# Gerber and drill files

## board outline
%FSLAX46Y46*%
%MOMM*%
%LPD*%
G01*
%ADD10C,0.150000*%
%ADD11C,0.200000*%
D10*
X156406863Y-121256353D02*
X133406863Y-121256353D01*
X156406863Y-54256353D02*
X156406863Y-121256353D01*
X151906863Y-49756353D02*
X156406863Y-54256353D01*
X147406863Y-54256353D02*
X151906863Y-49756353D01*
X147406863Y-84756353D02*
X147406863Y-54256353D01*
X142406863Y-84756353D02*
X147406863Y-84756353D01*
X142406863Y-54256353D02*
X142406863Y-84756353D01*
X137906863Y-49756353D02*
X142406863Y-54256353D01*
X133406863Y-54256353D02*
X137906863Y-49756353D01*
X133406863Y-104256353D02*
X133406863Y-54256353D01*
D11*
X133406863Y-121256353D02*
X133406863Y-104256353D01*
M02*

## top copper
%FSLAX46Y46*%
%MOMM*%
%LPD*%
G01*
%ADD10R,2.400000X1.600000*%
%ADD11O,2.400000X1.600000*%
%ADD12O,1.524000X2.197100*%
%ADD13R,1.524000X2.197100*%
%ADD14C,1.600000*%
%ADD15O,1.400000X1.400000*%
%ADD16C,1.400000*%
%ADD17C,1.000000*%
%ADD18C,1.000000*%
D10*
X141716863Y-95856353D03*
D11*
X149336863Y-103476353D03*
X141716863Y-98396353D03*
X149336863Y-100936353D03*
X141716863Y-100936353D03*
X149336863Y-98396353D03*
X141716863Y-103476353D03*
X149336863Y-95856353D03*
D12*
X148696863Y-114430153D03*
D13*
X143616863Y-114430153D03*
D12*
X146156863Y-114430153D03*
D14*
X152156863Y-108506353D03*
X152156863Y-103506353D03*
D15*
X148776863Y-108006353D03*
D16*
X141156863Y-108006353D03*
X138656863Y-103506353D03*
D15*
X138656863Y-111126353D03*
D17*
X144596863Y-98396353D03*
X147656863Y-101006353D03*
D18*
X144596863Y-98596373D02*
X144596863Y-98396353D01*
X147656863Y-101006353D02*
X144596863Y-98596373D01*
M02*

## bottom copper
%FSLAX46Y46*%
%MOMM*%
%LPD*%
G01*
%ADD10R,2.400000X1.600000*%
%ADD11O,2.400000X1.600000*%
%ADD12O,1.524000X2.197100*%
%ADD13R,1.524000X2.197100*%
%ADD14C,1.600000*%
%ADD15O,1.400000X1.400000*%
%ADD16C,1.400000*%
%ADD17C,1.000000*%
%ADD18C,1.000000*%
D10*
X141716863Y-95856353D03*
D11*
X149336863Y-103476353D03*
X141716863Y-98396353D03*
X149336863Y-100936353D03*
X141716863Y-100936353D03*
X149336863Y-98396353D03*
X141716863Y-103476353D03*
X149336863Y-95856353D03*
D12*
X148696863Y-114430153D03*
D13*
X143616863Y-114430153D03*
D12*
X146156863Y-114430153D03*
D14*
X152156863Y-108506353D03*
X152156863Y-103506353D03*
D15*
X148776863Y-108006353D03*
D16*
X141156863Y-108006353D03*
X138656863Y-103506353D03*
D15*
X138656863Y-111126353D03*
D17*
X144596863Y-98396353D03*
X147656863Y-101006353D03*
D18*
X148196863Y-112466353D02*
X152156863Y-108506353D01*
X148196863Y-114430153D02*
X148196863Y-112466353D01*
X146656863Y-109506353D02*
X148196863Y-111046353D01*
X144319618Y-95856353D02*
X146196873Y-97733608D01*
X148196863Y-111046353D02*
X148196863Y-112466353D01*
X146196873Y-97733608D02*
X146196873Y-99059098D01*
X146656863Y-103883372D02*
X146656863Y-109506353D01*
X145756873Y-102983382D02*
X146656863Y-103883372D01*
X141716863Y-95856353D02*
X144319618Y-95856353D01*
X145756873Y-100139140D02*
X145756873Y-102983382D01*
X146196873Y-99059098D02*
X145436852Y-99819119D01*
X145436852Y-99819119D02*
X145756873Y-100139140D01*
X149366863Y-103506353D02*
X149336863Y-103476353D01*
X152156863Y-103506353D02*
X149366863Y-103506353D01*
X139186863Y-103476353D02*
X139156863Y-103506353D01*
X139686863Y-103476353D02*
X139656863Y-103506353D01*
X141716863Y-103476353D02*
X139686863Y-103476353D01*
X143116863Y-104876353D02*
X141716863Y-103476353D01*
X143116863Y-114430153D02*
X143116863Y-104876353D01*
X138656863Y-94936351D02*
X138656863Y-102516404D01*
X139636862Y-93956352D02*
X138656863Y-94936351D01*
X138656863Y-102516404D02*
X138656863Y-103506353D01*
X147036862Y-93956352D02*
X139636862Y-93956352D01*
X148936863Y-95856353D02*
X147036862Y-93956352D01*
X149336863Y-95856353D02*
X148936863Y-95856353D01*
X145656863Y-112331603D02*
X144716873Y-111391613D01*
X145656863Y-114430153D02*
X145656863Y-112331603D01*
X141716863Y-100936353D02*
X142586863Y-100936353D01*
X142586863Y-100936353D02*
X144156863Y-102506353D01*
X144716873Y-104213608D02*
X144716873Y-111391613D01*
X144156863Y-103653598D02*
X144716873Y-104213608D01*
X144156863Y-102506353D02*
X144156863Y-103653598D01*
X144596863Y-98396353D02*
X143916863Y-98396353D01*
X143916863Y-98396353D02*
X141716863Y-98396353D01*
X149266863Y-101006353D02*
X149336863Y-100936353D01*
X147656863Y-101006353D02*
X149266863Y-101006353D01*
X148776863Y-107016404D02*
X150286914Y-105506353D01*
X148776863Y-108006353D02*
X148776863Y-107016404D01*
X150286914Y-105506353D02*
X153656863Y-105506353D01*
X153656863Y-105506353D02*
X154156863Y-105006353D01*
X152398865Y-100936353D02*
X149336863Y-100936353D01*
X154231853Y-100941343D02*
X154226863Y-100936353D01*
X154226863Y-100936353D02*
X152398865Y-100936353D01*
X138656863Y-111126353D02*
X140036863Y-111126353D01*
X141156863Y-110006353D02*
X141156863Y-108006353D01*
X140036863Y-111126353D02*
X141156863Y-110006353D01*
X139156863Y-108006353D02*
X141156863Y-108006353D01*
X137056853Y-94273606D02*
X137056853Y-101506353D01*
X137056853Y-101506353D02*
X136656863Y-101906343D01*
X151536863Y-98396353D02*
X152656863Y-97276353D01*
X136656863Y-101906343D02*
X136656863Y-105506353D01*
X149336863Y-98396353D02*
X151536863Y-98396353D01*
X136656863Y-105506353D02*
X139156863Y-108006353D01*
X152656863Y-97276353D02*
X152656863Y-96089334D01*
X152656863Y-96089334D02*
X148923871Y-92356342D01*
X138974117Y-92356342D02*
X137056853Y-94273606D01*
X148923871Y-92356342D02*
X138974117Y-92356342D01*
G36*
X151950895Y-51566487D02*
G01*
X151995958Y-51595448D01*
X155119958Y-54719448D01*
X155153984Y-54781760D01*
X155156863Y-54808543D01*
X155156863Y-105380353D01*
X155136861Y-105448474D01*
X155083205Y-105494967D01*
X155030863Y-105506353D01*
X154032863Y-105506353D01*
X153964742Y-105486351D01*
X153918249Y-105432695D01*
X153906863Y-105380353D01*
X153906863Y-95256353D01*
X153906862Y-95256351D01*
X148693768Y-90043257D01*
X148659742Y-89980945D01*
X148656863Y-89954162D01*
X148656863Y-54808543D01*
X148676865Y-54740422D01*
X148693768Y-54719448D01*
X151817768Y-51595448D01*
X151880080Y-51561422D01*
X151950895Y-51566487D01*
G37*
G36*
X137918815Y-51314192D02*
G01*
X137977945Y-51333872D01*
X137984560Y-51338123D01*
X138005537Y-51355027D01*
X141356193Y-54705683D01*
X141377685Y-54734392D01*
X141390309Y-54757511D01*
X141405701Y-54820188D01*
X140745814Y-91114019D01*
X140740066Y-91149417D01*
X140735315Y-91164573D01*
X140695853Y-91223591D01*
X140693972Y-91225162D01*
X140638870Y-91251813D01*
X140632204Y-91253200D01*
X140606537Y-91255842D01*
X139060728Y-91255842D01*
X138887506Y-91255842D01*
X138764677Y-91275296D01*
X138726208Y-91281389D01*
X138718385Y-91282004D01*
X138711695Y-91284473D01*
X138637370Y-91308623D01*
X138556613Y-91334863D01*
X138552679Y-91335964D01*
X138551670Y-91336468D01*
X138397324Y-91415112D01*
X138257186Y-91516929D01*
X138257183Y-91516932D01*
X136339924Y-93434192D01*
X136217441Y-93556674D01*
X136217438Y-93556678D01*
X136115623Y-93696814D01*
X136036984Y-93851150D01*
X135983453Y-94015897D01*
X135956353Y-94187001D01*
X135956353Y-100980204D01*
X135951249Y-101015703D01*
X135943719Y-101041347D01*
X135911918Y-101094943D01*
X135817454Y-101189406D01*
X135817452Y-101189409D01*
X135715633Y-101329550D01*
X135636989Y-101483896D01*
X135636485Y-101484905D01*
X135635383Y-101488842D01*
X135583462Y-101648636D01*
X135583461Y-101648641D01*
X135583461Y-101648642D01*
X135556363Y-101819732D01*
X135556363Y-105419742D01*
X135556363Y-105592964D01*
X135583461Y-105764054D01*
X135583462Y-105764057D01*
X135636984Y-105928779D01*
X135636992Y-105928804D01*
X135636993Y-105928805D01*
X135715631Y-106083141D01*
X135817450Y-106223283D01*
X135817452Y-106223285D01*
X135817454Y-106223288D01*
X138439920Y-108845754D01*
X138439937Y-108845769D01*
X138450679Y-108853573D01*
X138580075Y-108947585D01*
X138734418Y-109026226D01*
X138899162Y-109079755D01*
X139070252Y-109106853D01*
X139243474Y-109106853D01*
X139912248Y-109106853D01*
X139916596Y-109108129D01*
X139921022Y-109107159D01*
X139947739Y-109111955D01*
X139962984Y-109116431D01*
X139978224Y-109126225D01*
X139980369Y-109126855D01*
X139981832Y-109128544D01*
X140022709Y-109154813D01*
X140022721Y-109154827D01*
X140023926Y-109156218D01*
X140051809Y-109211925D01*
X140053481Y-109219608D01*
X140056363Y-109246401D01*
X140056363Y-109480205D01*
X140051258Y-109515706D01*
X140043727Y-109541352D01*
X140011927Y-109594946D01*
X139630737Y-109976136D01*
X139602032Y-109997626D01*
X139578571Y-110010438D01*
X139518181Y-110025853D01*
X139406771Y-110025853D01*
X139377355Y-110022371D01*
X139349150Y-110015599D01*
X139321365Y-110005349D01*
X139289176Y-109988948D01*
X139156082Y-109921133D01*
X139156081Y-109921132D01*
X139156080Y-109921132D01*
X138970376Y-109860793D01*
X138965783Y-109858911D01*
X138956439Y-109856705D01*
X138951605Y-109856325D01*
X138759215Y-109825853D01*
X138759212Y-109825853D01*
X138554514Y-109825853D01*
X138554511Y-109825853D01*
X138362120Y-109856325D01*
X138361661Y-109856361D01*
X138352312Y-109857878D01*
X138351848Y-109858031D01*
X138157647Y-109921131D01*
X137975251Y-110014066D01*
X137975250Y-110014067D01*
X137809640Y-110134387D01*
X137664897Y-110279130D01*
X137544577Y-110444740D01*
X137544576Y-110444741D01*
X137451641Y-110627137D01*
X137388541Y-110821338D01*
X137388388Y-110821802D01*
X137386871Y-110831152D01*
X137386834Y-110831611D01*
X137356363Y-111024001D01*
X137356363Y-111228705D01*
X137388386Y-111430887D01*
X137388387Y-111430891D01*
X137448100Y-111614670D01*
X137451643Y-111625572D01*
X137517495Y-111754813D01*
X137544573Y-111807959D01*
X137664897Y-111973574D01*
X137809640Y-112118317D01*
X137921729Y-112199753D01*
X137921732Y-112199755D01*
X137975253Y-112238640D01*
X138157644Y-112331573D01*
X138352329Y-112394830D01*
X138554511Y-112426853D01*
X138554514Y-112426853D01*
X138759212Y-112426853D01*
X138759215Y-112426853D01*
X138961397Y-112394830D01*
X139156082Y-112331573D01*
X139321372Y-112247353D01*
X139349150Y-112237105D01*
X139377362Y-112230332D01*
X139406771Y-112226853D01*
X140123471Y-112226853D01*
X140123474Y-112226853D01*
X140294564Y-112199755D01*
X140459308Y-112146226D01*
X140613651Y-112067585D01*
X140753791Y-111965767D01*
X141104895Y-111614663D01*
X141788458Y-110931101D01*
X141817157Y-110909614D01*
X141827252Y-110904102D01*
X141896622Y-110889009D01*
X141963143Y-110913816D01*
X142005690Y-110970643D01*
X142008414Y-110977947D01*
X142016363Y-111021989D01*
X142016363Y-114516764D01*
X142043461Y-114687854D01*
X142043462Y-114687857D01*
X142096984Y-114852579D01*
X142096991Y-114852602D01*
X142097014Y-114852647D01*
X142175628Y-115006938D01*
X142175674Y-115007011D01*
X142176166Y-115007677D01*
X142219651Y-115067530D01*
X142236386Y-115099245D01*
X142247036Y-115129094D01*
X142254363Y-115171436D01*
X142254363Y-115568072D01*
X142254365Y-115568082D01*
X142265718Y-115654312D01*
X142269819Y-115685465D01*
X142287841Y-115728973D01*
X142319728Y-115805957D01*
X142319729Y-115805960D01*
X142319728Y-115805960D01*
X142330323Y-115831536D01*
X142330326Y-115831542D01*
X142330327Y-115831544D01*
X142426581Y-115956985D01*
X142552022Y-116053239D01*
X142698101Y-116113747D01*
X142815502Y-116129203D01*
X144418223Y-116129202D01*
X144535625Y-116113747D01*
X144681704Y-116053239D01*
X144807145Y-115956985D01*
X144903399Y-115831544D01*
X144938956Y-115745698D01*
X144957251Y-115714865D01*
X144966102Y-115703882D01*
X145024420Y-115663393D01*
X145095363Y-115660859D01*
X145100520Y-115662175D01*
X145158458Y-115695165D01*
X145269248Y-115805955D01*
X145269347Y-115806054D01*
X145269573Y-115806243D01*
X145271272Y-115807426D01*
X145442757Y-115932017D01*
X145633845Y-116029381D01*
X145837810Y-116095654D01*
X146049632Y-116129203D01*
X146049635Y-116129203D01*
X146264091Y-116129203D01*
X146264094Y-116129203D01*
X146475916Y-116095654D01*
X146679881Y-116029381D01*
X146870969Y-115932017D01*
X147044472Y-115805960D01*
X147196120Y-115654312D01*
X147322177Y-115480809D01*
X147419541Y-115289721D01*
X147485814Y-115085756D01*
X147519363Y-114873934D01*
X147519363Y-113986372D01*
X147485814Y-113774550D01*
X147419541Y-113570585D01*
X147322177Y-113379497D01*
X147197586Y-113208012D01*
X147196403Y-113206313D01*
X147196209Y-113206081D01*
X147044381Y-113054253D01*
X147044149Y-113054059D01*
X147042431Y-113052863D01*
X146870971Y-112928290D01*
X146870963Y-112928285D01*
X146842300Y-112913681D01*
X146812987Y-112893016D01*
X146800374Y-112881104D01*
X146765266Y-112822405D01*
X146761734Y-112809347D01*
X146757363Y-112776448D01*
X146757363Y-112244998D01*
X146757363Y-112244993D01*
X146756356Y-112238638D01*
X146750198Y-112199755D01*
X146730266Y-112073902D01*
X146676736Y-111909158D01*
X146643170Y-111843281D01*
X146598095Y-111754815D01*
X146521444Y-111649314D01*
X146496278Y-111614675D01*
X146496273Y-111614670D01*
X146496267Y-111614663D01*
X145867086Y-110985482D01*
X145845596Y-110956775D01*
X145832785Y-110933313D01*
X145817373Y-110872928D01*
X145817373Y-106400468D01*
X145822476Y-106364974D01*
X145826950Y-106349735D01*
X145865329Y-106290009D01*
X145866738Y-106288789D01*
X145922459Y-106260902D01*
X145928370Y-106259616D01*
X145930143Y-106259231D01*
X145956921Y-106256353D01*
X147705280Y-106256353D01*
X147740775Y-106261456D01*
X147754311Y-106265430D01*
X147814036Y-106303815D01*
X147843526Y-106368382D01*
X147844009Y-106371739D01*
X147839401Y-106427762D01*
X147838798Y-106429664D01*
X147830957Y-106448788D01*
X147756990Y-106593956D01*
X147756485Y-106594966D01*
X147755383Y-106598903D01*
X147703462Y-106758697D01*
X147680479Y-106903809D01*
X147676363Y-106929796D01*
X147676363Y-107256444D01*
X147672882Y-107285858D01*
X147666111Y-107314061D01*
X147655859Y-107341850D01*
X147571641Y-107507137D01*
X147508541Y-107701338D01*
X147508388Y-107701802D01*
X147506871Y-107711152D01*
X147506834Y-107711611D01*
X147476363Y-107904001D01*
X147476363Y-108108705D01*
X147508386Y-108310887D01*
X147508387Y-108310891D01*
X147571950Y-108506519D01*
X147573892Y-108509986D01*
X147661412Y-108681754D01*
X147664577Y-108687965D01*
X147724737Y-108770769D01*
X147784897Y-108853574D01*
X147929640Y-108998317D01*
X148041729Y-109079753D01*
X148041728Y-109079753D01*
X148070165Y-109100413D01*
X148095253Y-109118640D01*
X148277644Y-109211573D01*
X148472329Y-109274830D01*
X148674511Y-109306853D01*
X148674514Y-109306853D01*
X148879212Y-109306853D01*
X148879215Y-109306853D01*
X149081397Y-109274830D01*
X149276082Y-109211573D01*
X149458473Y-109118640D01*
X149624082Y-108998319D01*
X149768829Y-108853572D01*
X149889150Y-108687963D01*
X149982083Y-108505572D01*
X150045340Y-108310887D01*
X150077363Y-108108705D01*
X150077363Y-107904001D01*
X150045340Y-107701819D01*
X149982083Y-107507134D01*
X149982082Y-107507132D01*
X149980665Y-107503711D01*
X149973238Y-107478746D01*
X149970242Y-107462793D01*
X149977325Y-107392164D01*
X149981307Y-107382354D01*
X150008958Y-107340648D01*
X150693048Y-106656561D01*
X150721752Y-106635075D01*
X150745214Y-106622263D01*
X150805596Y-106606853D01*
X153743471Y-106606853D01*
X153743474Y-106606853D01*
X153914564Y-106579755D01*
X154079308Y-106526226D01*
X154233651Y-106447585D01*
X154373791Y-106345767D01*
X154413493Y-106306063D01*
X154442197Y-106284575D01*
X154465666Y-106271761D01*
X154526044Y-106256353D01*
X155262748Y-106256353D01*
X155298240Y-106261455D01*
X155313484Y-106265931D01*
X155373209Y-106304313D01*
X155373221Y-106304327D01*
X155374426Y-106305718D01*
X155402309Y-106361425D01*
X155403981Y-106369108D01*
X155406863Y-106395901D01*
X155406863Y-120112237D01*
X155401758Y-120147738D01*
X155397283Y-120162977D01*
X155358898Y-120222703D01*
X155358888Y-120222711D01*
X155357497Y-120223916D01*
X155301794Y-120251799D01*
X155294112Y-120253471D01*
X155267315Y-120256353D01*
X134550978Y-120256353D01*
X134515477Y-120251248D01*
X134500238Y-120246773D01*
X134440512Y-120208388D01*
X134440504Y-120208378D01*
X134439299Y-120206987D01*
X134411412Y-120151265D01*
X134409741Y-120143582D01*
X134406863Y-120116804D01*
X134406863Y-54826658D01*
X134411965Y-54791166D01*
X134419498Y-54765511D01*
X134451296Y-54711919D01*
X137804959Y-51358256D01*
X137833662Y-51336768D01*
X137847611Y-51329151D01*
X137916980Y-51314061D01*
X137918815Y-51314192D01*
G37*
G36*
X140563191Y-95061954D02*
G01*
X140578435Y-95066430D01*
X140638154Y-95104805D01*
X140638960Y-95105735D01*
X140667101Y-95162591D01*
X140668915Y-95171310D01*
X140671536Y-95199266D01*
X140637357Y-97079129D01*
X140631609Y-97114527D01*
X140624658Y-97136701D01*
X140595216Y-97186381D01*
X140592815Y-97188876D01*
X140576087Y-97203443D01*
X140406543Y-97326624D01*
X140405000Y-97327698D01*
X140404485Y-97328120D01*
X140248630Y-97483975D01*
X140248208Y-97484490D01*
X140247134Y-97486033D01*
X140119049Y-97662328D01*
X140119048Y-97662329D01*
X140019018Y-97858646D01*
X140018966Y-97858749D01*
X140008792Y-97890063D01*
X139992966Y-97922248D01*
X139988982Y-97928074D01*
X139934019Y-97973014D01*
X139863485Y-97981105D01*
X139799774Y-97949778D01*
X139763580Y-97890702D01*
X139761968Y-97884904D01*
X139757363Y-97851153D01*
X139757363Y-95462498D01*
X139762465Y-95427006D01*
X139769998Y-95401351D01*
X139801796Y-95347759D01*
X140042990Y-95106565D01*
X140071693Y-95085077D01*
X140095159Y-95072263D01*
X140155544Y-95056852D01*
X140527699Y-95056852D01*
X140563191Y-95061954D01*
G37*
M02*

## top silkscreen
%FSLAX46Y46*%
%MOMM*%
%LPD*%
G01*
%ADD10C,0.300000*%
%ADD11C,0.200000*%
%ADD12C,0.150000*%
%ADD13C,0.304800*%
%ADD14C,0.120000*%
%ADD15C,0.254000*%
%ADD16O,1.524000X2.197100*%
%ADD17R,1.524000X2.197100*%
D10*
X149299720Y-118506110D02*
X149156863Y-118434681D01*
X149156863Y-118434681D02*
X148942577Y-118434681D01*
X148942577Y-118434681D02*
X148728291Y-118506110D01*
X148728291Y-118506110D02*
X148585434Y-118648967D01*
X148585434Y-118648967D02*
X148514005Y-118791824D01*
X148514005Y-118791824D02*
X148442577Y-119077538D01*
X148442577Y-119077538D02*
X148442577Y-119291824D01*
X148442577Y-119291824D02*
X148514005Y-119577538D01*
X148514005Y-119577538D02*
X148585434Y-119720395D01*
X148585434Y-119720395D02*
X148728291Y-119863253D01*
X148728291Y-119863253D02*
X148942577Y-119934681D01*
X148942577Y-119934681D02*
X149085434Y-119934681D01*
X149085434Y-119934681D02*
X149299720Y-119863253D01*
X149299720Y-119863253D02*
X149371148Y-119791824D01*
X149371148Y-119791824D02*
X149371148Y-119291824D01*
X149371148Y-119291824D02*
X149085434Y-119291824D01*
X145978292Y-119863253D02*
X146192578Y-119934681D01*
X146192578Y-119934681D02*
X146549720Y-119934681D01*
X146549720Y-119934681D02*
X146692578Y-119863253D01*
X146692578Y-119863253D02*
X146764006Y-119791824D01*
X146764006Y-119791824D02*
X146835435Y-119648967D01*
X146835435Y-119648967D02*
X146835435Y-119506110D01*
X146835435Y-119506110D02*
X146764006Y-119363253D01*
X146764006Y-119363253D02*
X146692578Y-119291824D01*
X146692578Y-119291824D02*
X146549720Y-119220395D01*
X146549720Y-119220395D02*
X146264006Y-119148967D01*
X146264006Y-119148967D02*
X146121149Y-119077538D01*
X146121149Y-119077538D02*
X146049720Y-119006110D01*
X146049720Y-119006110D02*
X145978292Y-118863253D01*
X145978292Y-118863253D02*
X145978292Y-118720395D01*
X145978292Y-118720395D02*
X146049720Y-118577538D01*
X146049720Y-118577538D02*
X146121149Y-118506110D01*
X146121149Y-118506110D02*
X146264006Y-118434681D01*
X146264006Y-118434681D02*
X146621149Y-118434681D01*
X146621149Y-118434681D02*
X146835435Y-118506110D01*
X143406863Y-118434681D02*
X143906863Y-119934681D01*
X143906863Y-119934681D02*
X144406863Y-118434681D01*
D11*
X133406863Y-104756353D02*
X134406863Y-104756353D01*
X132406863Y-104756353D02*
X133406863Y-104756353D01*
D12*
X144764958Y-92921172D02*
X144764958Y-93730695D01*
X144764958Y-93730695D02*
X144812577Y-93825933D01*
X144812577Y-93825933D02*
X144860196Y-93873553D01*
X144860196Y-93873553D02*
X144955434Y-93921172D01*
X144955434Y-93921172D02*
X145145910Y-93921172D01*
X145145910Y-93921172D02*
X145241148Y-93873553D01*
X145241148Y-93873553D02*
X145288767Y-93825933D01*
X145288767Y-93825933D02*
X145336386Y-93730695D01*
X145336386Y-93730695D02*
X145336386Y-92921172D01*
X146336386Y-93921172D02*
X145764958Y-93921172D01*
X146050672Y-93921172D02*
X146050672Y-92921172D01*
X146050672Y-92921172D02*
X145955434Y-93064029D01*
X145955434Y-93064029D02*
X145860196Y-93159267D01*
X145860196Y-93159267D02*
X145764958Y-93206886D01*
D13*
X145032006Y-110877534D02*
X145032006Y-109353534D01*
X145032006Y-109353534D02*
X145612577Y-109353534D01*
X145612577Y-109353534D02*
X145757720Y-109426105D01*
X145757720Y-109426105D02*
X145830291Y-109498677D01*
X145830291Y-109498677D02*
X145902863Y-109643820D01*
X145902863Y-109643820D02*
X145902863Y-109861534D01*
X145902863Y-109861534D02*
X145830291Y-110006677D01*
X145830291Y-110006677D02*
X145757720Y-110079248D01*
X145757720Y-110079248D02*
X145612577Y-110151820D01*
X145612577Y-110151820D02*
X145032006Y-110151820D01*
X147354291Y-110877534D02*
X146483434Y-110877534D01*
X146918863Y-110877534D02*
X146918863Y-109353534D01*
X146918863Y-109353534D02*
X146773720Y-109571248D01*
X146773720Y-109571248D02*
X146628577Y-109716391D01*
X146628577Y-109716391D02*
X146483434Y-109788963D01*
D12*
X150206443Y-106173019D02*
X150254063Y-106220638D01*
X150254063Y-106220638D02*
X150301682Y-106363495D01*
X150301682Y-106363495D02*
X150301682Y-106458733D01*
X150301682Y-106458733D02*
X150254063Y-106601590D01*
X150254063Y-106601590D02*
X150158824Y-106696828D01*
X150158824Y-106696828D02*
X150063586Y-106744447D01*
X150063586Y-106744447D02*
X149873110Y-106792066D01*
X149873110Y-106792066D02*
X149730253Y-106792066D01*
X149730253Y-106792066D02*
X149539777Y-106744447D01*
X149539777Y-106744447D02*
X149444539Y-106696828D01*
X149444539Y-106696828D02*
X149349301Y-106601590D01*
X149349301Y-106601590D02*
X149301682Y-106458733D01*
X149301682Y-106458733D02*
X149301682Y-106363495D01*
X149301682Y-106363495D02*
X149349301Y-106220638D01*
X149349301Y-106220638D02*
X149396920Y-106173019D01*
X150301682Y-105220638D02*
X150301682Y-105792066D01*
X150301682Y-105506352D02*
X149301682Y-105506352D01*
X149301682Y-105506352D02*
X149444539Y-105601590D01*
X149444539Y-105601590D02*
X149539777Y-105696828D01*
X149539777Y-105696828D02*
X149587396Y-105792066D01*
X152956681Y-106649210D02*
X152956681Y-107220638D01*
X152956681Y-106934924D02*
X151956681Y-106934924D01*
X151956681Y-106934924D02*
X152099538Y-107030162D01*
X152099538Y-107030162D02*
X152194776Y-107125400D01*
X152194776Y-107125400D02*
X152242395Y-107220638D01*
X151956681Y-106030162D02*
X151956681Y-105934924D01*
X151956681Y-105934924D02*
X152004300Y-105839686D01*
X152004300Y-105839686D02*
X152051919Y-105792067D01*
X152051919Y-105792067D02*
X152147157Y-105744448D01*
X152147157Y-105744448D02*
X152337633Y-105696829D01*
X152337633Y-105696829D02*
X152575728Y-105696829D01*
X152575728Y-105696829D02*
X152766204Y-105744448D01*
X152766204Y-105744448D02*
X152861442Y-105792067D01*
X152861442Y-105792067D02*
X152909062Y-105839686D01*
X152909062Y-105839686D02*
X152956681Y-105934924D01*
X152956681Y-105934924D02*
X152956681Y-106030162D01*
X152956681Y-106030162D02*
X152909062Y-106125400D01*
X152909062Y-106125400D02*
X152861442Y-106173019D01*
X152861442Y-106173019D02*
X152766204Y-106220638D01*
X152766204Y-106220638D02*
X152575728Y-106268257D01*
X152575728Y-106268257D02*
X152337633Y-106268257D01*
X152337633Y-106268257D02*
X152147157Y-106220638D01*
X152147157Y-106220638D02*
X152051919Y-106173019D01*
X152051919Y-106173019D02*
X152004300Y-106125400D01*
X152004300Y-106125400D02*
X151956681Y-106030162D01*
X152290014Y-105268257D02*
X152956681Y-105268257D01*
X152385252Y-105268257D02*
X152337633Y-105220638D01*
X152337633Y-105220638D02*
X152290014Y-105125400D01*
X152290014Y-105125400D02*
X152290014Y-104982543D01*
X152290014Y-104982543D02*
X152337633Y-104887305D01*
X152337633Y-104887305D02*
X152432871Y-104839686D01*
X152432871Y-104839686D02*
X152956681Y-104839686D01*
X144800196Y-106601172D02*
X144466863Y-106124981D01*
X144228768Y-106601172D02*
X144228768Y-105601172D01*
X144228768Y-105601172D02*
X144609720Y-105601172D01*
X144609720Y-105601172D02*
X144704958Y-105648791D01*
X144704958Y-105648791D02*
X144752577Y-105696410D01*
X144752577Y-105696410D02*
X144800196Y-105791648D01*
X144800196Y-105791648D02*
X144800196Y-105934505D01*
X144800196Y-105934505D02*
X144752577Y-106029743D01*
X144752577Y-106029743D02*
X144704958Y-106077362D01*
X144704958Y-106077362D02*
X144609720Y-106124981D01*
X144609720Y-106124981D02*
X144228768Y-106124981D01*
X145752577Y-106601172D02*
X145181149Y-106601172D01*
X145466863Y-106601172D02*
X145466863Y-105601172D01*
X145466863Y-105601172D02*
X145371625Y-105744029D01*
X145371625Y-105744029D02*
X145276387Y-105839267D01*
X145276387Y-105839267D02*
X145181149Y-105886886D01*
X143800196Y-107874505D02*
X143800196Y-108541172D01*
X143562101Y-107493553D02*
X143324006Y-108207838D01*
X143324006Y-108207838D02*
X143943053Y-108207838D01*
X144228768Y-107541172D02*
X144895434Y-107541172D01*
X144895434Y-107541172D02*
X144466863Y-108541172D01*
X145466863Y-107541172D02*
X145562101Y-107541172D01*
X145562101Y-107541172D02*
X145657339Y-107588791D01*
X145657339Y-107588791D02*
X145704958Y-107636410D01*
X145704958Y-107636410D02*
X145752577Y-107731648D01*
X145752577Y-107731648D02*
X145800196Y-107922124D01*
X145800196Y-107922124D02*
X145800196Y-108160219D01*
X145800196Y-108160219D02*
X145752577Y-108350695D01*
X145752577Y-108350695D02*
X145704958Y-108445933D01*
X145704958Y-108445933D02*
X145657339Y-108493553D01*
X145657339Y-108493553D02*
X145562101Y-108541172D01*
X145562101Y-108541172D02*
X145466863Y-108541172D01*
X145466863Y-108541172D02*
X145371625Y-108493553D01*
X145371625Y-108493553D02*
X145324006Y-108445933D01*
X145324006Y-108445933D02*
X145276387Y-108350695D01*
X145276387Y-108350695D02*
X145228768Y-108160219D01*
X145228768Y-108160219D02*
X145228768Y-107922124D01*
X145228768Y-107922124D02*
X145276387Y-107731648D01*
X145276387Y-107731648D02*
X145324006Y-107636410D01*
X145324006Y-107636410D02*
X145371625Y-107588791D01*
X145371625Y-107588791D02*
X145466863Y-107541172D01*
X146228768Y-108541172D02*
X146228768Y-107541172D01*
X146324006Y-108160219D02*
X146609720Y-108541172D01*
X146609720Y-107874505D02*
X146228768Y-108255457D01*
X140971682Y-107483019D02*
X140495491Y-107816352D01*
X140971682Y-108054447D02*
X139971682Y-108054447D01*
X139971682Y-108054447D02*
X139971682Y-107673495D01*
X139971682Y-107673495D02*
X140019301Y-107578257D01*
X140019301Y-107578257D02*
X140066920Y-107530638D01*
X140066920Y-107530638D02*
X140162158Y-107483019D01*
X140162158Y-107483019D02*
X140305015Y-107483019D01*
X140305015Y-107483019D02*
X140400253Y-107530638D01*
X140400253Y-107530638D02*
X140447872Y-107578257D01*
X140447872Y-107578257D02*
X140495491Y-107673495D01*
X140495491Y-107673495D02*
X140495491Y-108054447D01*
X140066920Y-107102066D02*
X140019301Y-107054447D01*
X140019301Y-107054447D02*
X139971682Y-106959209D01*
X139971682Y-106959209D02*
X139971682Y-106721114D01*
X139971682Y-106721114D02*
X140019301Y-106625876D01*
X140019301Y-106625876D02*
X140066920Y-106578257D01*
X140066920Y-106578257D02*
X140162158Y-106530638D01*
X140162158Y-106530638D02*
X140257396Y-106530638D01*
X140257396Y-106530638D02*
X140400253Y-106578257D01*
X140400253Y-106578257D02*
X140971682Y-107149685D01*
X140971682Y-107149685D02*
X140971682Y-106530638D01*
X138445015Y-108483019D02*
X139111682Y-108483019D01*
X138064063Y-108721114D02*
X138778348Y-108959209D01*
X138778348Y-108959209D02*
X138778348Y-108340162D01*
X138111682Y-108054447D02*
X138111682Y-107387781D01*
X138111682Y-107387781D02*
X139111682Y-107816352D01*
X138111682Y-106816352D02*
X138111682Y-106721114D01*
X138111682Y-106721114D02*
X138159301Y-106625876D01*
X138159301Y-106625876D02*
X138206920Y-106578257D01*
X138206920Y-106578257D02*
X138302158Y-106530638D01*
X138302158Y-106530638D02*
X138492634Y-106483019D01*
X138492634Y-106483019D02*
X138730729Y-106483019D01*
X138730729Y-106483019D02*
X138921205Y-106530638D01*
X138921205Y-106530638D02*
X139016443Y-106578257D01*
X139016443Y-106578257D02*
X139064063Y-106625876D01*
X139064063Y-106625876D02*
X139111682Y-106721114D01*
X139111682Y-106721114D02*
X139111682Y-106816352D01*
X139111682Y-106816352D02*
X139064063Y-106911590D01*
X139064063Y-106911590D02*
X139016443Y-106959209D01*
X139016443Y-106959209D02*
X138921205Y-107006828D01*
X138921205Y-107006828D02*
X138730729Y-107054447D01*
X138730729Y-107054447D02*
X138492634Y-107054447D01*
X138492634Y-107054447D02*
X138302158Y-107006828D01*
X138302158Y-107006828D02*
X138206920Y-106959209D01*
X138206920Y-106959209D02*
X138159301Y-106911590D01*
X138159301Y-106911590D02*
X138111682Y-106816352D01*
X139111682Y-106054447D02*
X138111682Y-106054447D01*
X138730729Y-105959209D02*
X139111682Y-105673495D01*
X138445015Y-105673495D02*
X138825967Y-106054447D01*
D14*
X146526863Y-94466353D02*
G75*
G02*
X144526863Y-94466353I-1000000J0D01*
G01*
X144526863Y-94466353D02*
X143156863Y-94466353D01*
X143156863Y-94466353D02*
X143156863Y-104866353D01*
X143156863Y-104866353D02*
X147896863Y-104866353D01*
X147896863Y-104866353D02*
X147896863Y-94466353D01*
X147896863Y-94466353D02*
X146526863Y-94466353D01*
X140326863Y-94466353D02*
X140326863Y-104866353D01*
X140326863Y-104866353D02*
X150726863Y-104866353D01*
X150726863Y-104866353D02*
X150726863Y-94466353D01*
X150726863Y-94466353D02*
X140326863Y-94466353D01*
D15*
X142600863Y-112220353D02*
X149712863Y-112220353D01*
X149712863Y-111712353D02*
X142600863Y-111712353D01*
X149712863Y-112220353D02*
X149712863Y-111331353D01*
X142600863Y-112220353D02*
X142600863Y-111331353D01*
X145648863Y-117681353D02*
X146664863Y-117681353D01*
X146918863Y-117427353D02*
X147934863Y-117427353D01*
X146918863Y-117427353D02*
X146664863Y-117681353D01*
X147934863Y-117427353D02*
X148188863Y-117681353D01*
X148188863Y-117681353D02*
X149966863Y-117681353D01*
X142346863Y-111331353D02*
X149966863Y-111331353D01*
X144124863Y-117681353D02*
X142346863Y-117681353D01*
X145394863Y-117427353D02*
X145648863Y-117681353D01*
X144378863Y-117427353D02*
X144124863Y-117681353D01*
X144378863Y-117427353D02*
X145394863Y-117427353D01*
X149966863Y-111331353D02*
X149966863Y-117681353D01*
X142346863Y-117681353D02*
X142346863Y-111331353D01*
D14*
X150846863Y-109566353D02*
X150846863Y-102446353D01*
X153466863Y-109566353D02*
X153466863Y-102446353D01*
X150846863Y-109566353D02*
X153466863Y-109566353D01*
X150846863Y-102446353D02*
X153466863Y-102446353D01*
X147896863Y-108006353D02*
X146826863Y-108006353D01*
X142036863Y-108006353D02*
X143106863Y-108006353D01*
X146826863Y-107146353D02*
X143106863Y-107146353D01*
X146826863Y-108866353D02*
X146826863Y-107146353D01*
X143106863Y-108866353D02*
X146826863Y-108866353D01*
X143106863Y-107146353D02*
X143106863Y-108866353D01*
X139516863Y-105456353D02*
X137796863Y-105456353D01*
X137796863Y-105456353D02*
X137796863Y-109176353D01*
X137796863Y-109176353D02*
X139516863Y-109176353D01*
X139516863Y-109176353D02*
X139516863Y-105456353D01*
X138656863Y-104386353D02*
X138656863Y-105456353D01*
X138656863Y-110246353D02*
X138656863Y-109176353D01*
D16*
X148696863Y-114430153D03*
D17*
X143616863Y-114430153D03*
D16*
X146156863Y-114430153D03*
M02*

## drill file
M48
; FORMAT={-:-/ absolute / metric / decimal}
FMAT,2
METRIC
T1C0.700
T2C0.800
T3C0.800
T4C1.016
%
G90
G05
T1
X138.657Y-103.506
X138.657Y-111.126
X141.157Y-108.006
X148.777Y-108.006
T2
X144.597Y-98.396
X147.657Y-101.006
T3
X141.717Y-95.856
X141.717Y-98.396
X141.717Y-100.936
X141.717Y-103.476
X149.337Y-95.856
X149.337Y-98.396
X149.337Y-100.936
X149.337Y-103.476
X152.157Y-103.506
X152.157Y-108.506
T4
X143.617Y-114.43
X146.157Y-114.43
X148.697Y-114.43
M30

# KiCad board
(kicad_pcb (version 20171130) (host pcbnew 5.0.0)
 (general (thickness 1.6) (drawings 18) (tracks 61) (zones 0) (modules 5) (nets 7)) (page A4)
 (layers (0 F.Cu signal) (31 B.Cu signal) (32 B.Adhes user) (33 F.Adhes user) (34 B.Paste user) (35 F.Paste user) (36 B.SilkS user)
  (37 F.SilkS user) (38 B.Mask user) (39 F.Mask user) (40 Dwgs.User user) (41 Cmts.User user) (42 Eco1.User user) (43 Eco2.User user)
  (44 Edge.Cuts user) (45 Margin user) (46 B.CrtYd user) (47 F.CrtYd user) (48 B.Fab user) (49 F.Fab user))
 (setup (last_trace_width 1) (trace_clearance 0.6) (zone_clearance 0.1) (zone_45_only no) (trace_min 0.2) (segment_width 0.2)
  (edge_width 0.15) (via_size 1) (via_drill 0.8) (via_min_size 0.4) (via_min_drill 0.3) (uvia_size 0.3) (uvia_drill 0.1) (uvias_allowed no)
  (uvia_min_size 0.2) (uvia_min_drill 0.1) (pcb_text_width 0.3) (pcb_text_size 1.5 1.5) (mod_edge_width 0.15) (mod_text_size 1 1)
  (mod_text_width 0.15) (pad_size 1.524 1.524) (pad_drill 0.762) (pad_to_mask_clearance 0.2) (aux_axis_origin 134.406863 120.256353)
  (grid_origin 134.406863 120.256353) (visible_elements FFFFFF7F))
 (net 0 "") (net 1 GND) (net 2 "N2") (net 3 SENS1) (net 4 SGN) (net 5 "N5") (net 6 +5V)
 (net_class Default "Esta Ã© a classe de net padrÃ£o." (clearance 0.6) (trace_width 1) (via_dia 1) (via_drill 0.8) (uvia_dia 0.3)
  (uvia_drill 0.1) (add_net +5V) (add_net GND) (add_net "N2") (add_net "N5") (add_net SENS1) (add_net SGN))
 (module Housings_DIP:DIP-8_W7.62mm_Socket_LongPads (layer F.Cu) (at 141.716863 95.856353)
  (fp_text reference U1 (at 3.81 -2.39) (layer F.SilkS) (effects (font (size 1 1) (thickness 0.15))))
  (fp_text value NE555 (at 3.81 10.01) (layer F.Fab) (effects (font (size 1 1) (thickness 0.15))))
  (fp_arc (start 3.81 -1.39) (end 2.81 -1.39) (angle -180) (layer F.SilkS) (width 0.12))
  (fp_line (start 2.81 -1.39) (end 1.44 -1.39) (layer F.SilkS) (width 0.12))
  (fp_line (start 1.44 -1.39) (end 1.44 9.01) (layer F.SilkS) (width 0.12))
  (fp_line (start 1.44 9.01) (end 6.18 9.01) (layer F.SilkS) (width 0.12))
  (fp_line (start 6.18 9.01) (end 6.18 -1.39) (layer F.SilkS) (width 0.12))
  (fp_line (start 6.18 -1.39) (end 4.81 -1.39) (layer F.SilkS) (width 0.12))
  (fp_line (start -1.39 -1.39) (end -1.39 9.01) (layer F.SilkS) (width 0.12))
  (fp_line (start -1.39 9.01) (end 9.01 9.01) (layer F.SilkS) (width 0.12))
  (fp_line (start 9.01 9.01) (end 9.01 -1.39) (layer F.SilkS) (width 0.12))
  (fp_line (start 9.01 -1.39) (end -1.39 -1.39) (layer F.SilkS) (width 0.12))
  (pad 1 thru_hole rect (at 0 0) (size 2.4 1.6) (drill 0.8) (layers *.Mask B.Cu) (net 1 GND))
  (pad 5 thru_hole oval (at 7.62 7.62) (size 2.4 1.6) (drill 0.8) (layers *.Mask B.Cu) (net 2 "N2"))
  (pad 2 thru_hole oval (at 0 2.54) (size 2.4 1.6) (drill 0.8) (layers *.Mask B.Cu) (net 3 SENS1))
  (pad 6 thru_hole oval (at 7.62 5.08) (size 2.4 1.6) (drill 0.8) (layers *.Mask B.Cu) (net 3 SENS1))
  (pad 3 thru_hole oval (at 0 5.08) (size 2.4 1.6) (drill 0.8) (layers *.Mask B.Cu) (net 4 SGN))
  (pad 7 thru_hole oval (at 7.62 2.54) (size 2.4 1.6) (drill 0.8) (layers *.Mask B.Cu) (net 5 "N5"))
  (pad 4 thru_hole oval (at 0 7.62) (size 2.4 1.6) (drill 0.8) (layers *.Mask B.Cu) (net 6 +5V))
  (pad 8 thru_hole oval (at 7.62 0) (size 2.4 1.6) (drill 0.8) (layers *.Mask B.Cu) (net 6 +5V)))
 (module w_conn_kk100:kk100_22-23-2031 (layer F.Cu) (at 146.156863 114.506353)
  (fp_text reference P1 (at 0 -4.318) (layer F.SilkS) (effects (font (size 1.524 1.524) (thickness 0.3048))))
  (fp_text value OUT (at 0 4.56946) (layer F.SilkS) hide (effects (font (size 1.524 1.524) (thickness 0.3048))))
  (fp_line (start -3.556 -2.286) (end 3.556 -2.286) (layer F.SilkS) (width 0.254))
  (fp_line (start 3.556 -2.794) (end -3.556 -2.794) (layer F.SilkS) (width 0.254))
  (fp_line (start 3.556 -2.286) (end 3.556 -3.175) (layer F.SilkS) (width 0.254))
  (fp_line (start -3.556 -2.286) (end -3.556 -3.175) (layer F.SilkS) (width 0.254))
  (fp_line (start -0.508 3.175) (end 0.508 3.175) (layer F.SilkS) (width 0.254))
  (fp_line (start 0.762 2.921) (end 1.778 2.921) (layer F.SilkS) (width 0.254))
  (fp_line (start 0.762 2.921) (end 0.508 3.175) (layer F.SilkS) (width 0.254))
  (fp_line (start 1.778 2.921) (end 2.032 3.175) (layer F.SilkS) (width 0.254))
  (fp_line (start 2.032 3.175) (end 3.81 3.175) (layer F.SilkS) (width 0.254))
  (fp_line (start -3.81 -3.175) (end 3.81 -3.175) (layer F.SilkS) (width 0.254))
  (fp_line (start -2.032 3.175) (end -3.81 3.175) (layer F.SilkS) (width 0.254))
  (fp_line (start -0.762 2.921) (end -0.508 3.175) (layer F.SilkS) (width 0.254))
  (fp_line (start -1.778 2.921) (end -2.032 3.175) (layer F.SilkS) (width 0.254))
  (fp_line (start -1.778 2.921) (end -0.762 2.921) (layer F.SilkS) (width 0.254))
  (fp_line (start 3.81 -3.175) (end 3.81 3.175) (layer F.SilkS) (width 0.254))
  (fp_line (start -3.81 3.175) (end -3.81 -3.175) (layer F.SilkS) (width 0.254))
  (pad 3 thru_hole oval (at 2.54 -0.0762) (size 1.524 2.1971) (drill 1.016) (layers *.Cu *.Mask F.SilkS) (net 1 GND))
  (pad 1 thru_hole rect (at -2.54 -0.0762) (size 1.524 2.1971) (drill 1.016) (layers *.Cu *.Mask F.SilkS) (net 6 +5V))
  (pad 2 thru_hole oval (at 0 -0.0762) (size 1.524 2.1971) (drill 1.016) (layers *.Cu *.Mask F.SilkS) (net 4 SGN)))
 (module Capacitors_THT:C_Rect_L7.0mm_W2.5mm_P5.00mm (layer F.Cu) (at 152.156863 108.506353 90)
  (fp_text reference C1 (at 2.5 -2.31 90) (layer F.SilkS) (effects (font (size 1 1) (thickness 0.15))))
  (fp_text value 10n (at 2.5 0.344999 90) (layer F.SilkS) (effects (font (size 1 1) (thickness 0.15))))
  (fp_line (start -1.06 -1.31) (end 6.06 -1.31) (layer F.SilkS) (width 0.12))
  (fp_line (start -1.06 1.31) (end 6.06 1.31) (layer F.SilkS) (width 0.12))
  (fp_line (start -1.06 -1.31) (end -1.06 1.31) (layer F.SilkS) (width 0.12))
  (fp_line (start 6.06 -1.31) (end 6.06 1.31) (layer F.SilkS) (width 0.12))
  (pad 1 thru_hole circle (at 0 0 90) (size 1.6 1.6) (drill 0.8) (layers *.Mask B.Cu) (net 1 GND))
  (pad 2 thru_hole circle (at 5 0 90) (size 1.6 1.6) (drill 0.8) (layers *.Mask B.Cu) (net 2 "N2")))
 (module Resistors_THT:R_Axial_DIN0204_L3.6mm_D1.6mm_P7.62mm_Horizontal (layer F.Cu) (at 141.156863 108.006353)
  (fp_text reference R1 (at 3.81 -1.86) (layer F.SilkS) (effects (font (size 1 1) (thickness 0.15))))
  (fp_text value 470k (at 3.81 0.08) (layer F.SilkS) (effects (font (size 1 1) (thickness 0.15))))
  (fp_line (start 6.74 0) (end 5.67 0) (layer F.SilkS) (width 0.12))
  (fp_line (start 0.88 0) (end 1.95 0) (layer F.SilkS) (width 0.12))
  (fp_line (start 5.67 -0.86) (end 1.95 -0.86) (layer F.SilkS) (width 0.12))
  (fp_line (start 5.67 0.86) (end 5.67 -0.86) (layer F.SilkS) (width 0.12))
  (fp_line (start 1.95 0.86) (end 5.67 0.86) (layer F.SilkS) (width 0.12))
  (fp_line (start 1.95 -0.86) (end 1.95 0.86) (layer F.SilkS) (width 0.12))
  (pad 2 thru_hole oval (at 7.62 0) (size 1.4 1.4) (drill 0.7) (layers *.Cu *.Mask) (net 3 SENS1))
  (pad 1 thru_hole circle (at 0 0) (size 1.4 1.4) (drill 0.7) (layers *.Cu *.Mask) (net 5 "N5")))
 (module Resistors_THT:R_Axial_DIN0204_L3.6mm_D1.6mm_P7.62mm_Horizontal (layer F.Cu) (at 138.656863 103.506353 270)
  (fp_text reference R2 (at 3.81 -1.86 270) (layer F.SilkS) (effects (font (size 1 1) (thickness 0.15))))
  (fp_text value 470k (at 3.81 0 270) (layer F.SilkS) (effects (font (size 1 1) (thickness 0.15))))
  (fp_line (start 1.95 -0.86) (end 1.95 0.86) (layer F.SilkS) (width 0.12))
  (fp_line (start 1.95 0.86) (end 5.67 0.86) (layer F.SilkS) (width 0.12))
  (fp_line (start 5.67 0.86) (end 5.67 -0.86) (layer F.SilkS) (width 0.12))
  (fp_line (start 5.67 -0.86) (end 1.95 -0.86) (layer F.SilkS) (width 0.12))
  (fp_line (start 0.88 0) (end 1.95 0) (layer F.SilkS) (width 0.12))
  (fp_line (start 6.74 0) (end 5.67 0) (layer F.SilkS) (width 0.12))
  (pad 1 thru_hole circle (at 0 0 270) (size 1.4 1.4) (drill 0.7) (layers *.Cu *.Mask) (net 6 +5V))
  (pad 2 thru_hole oval (at 7.62 0 270) (size 1.4 1.4) (drill 0.7) (layers *.Cu *.Mask) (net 5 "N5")))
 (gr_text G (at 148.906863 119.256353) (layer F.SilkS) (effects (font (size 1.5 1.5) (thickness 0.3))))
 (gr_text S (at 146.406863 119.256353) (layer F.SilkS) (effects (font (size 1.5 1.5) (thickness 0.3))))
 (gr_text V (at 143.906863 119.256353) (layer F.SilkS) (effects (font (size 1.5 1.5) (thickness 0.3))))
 (gr_line (start 156.406863 121.256353) (end 133.406863 121.256353) (layer Edge.Cuts) (width 0.15))
 (gr_line (start 156.406863 54.256353) (end 156.406863 121.256353) (layer Edge.Cuts) (width 0.15))
 (gr_line (start 151.906863 49.756353) (end 156.406863 54.256353) (layer Edge.Cuts) (width 0.15))
 (gr_line (start 147.406863 54.256353) (end 151.906863 49.756353) (layer Edge.Cuts) (width 0.15))
 (gr_line (start 147.406863 84.756353) (end 147.406863 54.256353) (layer Edge.Cuts) (width 0.15))
 (gr_line (start 142.406863 84.756353) (end 147.406863 84.756353) (layer Edge.Cuts) (width 0.15))
 (gr_line (start 142.406863 54.256353) (end 142.406863 84.756353) (layer Edge.Cuts) (width 0.15))
 (gr_line (start 137.906863 49.756353) (end 142.406863 54.256353) (layer Edge.Cuts) (width 0.15))
 (gr_line (start 133.406863 54.256353) (end 137.906863 49.756353) (layer Edge.Cuts) (width 0.15))
 (gr_line (start 133.406863 104.256353) (end 133.406863 54.256353) (layer Edge.Cuts) (width 0.15))
 (gr_line (start 133.406863 121.256353) (end 133.406863 104.256353) (layer Edge.Cuts) (width 0.2))
 (gr_line (start 133.406863 104.756353) (end 134.406863 104.756353) (layer F.SilkS) (width 0.2))
 (gr_line (start 132.406863 104.756353) (end 133.406863 104.756353) (layer F.SilkS) (width 0.2))
 (segment (start 148.196863 112.466353) (end 152.156863 108.506353) (width 1) (layer B.Cu) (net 1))
 (segment (start 148.196863 114.430153) (end 148.196863 112.466353) (width 1) (layer B.Cu) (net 1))
 (segment (start 146.656863 109.506353) (end 148.196863 111.046353) (width 1) (layer B.Cu) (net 1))
 (segment (start 144.319618 95.856353) (end 146.196873 97.733608) (width 1) (layer B.Cu) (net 1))
 (segment (start 148.196863 111.046353) (end 148.196863 112.466353) (width 1) (layer B.Cu) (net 1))
 (segment (start 146.196873 97.733608) (end 146.196873 99.059098) (width 1) (layer B.Cu) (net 1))
 (segment (start 146.656863 103.883372) (end 146.656863 109.506353) (width 1) (layer B.Cu) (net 1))
 (segment (start 145.756873 102.983382) (end 146.656863 103.883372) (width 1) (layer B.Cu) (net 1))
 (segment (start 141.716863 95.856353) (end 144.319618 95.856353) (width 1) (layer B.Cu) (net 1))
 (segment (start 145.756873 100.13914) (end 145.756873 102.983382) (width 1) (layer B.Cu) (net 1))
 (segment (start 146.196873 99.059098) (end 145.436852 99.819119) (width 1) (layer B.Cu) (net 1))
 (segment (start 145.436852 99.819119) (end 145.756873 100.13914) (width 1) (layer B.Cu) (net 1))
 (segment (start 149.366863 103.506353) (end 149.336863 103.476353) (width 1) (layer B.Cu) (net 2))
 (segment (start 152.156863 103.506353) (end 149.366863 103.506353) (width 1) (layer B.Cu) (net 2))
 (segment (start 139.186863 103.476353) (end 139.156863 103.506353) (width 1) (layer B.Cu) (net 6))
 (segment (start 139.686863 103.476353) (end 139.656863 103.506353) (width 1) (layer B.Cu) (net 6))
 (segment (start 141.716863 103.476353) (end 139.686863 103.476353) (width 1) (layer B.Cu) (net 6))
 (segment (start 143.116863 104.876353) (end 141.716863 103.476353) (width 1) (layer B.Cu) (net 6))
 (segment (start 143.116863 114.430153) (end 143.116863 104.876353) (width 1) (layer B.Cu) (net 6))
 (segment (start 138.656863 94.936351) (end 138.656863 102.516404) (width 1) (layer B.Cu) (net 6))
 (segment (start 139.636862 93.956352) (end 138.656863 94.936351) (width 1) (layer B.Cu) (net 6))
 (segment (start 138.656863 102.516404) (end 138.656863 103.506353) (width 1) (layer B.Cu) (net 6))
 (segment (start 147.036862 93.956352) (end 139.636862 93.956352) (width 1) (layer B.Cu) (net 6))
 (segment (start 148.936863 95.856353) (end 147.036862 93.956352) (width 1) (layer B.Cu) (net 6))
 (segment (start 149.336863 95.856353) (end 148.936863 95.856353) (width 1) (layer B.Cu) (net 6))
 (segment (start 145.656863 112.331603) (end 144.716873 111.391613) (width 1) (layer B.Cu) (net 4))
 (segment (start 145.656863 114.430153) (end 145.656863 112.331603) (width 1) (layer B.Cu) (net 4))
 (segment (start 141.716863 100.936353) (end 142.586863 100.936353) (width 1) (layer B.Cu) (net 4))
 (segment (start 142.586863 100.936353) (end 144.156863 102.506353) (width 1) (layer B.Cu) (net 4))
 (segment (start 144.716873 104.213608) (end 144.716873 111.391613) (width 1) (layer B.Cu) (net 4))
 (segment (start 144.156863 103.653598) (end 144.716873 104.213608) (width 1) (layer B.Cu) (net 4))
 (segment (start 144.156863 102.506353) (end 144.156863 103.653598) (width 1) (layer B.Cu) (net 4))
 (segment (start 144.596863 98.396353) (end 143.916863 98.396353) (width 1) (layer B.Cu) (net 3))
 (segment (start 143.916863 98.396353) (end 141.716863 98.396353) (width 1) (layer B.Cu) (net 3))
 (via (at 144.596863 98.396353) (size 1) (drill 0.8) (layers F.Cu B.Cu) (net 3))
 (segment (start 144.596863 98.596373) (end 144.596863 98.396353) (width 1) (layer F.Cu) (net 3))
 (via (at 147.656863 101.006353) (size 1) (drill 0.8) (layers F.Cu B.Cu) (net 3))
 (segment (start 147.656863 101.006353) (end 144.596863 98.596373) (width 1) (layer F.Cu) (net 3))
 (segment (start 149.266863 101.006353) (end 149.336863 100.936353) (width 1) (layer B.Cu) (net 3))
 (segment (start 147.656863 101.006353) (end 149.266863 101.006353) (width 1) (layer B.Cu) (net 3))
 (segment (start 148.776863 107.016404) (end 150.286914 105.506353) (width 1) (layer B.Cu) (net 3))
 (segment (start 148.776863 108.006353) (end 148.776863 107.016404) (width 1) (layer B.Cu) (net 3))
 (segment (start 150.286914 105.506353) (end 153.656863 105.506353) (width 1) (layer B.Cu) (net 3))
 (segment (start 153.656863 105.506353) (end 154.156863 105.006353) (width 1) (layer B.Cu) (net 3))
 (segment (start 152.398865 100.936353) (end 149.336863 100.936353) (width 1) (layer B.Cu) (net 3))
 (segment (start 154.231853 100.941343) (end 154.226863 100.936353) (width 1) (layer B.Cu) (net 3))
 (segment (start 154.226863 100.936353) (end 152.398865 100.936353) (width 1) (layer B.Cu) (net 3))
 (segment (start 138.656863 111.126353) (end 140.036863 111.126353) (width 1) (layer B.Cu) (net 5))
 (segment (start 141.156863 110.006353) (end 141.156863 108.006353) (width 1) (layer B.Cu) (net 5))
 (segment (start 140.036863 111.126353) (end 141.156863 110.006353) (width 1) (layer B.Cu) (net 5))
 (segment (start 139.156863 108.006353) (end 141.156863 108.006353) (width 1) (layer B.Cu) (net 5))
 (segment (start 137.056853 94.273606) (end 137.056853 101.506353) (width 1) (layer B.Cu) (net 5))
 (segment (start 137.056853 101.506353) (end 136.656863 101.906343) (width 1) (layer B.Cu) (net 5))
 (segment (start 151.536863 98.396353) (end 152.656863 97.276353) (width 1) (layer B.Cu) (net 5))
 (segment (start 136.656863 101.906343) (end 136.656863 105.506353) (width 1) (layer B.Cu) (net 5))
 (segment (start 149.336863 98.396353) (end 151.536863 98.396353) (width 1) (layer B.Cu) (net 5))
 (segment (start 136.656863 105.506353) (end 139.156863 108.006353) (width 1) (layer B.Cu) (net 5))
 (segment (start 152.656863 97.276353) (end 152.656863 96.089334) (width 1) (layer B.Cu) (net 5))
 (segment (start 152.656863 96.089334) (end 148.923871 92.356342) (width 1) (layer B.Cu) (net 5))
 (segment (start 138.974117 92.356342) (end 137.056853 94.273606) (width 1) (layer B.Cu) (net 5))
 (segment (start 148.923871 92.356342) (end 138.974117 92.356342) (width 1) (layer B.Cu) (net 5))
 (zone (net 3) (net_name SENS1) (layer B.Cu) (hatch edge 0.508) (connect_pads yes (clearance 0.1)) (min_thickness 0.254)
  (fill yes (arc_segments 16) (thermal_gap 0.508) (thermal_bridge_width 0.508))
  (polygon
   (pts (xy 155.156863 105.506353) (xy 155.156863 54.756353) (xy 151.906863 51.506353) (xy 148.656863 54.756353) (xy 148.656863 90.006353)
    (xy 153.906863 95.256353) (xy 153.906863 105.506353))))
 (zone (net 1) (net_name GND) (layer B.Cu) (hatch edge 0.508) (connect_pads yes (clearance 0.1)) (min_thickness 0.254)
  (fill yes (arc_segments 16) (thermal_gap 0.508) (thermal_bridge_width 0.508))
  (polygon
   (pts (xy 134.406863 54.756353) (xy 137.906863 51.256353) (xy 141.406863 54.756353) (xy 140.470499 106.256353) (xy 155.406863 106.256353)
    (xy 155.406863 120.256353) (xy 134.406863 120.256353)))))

